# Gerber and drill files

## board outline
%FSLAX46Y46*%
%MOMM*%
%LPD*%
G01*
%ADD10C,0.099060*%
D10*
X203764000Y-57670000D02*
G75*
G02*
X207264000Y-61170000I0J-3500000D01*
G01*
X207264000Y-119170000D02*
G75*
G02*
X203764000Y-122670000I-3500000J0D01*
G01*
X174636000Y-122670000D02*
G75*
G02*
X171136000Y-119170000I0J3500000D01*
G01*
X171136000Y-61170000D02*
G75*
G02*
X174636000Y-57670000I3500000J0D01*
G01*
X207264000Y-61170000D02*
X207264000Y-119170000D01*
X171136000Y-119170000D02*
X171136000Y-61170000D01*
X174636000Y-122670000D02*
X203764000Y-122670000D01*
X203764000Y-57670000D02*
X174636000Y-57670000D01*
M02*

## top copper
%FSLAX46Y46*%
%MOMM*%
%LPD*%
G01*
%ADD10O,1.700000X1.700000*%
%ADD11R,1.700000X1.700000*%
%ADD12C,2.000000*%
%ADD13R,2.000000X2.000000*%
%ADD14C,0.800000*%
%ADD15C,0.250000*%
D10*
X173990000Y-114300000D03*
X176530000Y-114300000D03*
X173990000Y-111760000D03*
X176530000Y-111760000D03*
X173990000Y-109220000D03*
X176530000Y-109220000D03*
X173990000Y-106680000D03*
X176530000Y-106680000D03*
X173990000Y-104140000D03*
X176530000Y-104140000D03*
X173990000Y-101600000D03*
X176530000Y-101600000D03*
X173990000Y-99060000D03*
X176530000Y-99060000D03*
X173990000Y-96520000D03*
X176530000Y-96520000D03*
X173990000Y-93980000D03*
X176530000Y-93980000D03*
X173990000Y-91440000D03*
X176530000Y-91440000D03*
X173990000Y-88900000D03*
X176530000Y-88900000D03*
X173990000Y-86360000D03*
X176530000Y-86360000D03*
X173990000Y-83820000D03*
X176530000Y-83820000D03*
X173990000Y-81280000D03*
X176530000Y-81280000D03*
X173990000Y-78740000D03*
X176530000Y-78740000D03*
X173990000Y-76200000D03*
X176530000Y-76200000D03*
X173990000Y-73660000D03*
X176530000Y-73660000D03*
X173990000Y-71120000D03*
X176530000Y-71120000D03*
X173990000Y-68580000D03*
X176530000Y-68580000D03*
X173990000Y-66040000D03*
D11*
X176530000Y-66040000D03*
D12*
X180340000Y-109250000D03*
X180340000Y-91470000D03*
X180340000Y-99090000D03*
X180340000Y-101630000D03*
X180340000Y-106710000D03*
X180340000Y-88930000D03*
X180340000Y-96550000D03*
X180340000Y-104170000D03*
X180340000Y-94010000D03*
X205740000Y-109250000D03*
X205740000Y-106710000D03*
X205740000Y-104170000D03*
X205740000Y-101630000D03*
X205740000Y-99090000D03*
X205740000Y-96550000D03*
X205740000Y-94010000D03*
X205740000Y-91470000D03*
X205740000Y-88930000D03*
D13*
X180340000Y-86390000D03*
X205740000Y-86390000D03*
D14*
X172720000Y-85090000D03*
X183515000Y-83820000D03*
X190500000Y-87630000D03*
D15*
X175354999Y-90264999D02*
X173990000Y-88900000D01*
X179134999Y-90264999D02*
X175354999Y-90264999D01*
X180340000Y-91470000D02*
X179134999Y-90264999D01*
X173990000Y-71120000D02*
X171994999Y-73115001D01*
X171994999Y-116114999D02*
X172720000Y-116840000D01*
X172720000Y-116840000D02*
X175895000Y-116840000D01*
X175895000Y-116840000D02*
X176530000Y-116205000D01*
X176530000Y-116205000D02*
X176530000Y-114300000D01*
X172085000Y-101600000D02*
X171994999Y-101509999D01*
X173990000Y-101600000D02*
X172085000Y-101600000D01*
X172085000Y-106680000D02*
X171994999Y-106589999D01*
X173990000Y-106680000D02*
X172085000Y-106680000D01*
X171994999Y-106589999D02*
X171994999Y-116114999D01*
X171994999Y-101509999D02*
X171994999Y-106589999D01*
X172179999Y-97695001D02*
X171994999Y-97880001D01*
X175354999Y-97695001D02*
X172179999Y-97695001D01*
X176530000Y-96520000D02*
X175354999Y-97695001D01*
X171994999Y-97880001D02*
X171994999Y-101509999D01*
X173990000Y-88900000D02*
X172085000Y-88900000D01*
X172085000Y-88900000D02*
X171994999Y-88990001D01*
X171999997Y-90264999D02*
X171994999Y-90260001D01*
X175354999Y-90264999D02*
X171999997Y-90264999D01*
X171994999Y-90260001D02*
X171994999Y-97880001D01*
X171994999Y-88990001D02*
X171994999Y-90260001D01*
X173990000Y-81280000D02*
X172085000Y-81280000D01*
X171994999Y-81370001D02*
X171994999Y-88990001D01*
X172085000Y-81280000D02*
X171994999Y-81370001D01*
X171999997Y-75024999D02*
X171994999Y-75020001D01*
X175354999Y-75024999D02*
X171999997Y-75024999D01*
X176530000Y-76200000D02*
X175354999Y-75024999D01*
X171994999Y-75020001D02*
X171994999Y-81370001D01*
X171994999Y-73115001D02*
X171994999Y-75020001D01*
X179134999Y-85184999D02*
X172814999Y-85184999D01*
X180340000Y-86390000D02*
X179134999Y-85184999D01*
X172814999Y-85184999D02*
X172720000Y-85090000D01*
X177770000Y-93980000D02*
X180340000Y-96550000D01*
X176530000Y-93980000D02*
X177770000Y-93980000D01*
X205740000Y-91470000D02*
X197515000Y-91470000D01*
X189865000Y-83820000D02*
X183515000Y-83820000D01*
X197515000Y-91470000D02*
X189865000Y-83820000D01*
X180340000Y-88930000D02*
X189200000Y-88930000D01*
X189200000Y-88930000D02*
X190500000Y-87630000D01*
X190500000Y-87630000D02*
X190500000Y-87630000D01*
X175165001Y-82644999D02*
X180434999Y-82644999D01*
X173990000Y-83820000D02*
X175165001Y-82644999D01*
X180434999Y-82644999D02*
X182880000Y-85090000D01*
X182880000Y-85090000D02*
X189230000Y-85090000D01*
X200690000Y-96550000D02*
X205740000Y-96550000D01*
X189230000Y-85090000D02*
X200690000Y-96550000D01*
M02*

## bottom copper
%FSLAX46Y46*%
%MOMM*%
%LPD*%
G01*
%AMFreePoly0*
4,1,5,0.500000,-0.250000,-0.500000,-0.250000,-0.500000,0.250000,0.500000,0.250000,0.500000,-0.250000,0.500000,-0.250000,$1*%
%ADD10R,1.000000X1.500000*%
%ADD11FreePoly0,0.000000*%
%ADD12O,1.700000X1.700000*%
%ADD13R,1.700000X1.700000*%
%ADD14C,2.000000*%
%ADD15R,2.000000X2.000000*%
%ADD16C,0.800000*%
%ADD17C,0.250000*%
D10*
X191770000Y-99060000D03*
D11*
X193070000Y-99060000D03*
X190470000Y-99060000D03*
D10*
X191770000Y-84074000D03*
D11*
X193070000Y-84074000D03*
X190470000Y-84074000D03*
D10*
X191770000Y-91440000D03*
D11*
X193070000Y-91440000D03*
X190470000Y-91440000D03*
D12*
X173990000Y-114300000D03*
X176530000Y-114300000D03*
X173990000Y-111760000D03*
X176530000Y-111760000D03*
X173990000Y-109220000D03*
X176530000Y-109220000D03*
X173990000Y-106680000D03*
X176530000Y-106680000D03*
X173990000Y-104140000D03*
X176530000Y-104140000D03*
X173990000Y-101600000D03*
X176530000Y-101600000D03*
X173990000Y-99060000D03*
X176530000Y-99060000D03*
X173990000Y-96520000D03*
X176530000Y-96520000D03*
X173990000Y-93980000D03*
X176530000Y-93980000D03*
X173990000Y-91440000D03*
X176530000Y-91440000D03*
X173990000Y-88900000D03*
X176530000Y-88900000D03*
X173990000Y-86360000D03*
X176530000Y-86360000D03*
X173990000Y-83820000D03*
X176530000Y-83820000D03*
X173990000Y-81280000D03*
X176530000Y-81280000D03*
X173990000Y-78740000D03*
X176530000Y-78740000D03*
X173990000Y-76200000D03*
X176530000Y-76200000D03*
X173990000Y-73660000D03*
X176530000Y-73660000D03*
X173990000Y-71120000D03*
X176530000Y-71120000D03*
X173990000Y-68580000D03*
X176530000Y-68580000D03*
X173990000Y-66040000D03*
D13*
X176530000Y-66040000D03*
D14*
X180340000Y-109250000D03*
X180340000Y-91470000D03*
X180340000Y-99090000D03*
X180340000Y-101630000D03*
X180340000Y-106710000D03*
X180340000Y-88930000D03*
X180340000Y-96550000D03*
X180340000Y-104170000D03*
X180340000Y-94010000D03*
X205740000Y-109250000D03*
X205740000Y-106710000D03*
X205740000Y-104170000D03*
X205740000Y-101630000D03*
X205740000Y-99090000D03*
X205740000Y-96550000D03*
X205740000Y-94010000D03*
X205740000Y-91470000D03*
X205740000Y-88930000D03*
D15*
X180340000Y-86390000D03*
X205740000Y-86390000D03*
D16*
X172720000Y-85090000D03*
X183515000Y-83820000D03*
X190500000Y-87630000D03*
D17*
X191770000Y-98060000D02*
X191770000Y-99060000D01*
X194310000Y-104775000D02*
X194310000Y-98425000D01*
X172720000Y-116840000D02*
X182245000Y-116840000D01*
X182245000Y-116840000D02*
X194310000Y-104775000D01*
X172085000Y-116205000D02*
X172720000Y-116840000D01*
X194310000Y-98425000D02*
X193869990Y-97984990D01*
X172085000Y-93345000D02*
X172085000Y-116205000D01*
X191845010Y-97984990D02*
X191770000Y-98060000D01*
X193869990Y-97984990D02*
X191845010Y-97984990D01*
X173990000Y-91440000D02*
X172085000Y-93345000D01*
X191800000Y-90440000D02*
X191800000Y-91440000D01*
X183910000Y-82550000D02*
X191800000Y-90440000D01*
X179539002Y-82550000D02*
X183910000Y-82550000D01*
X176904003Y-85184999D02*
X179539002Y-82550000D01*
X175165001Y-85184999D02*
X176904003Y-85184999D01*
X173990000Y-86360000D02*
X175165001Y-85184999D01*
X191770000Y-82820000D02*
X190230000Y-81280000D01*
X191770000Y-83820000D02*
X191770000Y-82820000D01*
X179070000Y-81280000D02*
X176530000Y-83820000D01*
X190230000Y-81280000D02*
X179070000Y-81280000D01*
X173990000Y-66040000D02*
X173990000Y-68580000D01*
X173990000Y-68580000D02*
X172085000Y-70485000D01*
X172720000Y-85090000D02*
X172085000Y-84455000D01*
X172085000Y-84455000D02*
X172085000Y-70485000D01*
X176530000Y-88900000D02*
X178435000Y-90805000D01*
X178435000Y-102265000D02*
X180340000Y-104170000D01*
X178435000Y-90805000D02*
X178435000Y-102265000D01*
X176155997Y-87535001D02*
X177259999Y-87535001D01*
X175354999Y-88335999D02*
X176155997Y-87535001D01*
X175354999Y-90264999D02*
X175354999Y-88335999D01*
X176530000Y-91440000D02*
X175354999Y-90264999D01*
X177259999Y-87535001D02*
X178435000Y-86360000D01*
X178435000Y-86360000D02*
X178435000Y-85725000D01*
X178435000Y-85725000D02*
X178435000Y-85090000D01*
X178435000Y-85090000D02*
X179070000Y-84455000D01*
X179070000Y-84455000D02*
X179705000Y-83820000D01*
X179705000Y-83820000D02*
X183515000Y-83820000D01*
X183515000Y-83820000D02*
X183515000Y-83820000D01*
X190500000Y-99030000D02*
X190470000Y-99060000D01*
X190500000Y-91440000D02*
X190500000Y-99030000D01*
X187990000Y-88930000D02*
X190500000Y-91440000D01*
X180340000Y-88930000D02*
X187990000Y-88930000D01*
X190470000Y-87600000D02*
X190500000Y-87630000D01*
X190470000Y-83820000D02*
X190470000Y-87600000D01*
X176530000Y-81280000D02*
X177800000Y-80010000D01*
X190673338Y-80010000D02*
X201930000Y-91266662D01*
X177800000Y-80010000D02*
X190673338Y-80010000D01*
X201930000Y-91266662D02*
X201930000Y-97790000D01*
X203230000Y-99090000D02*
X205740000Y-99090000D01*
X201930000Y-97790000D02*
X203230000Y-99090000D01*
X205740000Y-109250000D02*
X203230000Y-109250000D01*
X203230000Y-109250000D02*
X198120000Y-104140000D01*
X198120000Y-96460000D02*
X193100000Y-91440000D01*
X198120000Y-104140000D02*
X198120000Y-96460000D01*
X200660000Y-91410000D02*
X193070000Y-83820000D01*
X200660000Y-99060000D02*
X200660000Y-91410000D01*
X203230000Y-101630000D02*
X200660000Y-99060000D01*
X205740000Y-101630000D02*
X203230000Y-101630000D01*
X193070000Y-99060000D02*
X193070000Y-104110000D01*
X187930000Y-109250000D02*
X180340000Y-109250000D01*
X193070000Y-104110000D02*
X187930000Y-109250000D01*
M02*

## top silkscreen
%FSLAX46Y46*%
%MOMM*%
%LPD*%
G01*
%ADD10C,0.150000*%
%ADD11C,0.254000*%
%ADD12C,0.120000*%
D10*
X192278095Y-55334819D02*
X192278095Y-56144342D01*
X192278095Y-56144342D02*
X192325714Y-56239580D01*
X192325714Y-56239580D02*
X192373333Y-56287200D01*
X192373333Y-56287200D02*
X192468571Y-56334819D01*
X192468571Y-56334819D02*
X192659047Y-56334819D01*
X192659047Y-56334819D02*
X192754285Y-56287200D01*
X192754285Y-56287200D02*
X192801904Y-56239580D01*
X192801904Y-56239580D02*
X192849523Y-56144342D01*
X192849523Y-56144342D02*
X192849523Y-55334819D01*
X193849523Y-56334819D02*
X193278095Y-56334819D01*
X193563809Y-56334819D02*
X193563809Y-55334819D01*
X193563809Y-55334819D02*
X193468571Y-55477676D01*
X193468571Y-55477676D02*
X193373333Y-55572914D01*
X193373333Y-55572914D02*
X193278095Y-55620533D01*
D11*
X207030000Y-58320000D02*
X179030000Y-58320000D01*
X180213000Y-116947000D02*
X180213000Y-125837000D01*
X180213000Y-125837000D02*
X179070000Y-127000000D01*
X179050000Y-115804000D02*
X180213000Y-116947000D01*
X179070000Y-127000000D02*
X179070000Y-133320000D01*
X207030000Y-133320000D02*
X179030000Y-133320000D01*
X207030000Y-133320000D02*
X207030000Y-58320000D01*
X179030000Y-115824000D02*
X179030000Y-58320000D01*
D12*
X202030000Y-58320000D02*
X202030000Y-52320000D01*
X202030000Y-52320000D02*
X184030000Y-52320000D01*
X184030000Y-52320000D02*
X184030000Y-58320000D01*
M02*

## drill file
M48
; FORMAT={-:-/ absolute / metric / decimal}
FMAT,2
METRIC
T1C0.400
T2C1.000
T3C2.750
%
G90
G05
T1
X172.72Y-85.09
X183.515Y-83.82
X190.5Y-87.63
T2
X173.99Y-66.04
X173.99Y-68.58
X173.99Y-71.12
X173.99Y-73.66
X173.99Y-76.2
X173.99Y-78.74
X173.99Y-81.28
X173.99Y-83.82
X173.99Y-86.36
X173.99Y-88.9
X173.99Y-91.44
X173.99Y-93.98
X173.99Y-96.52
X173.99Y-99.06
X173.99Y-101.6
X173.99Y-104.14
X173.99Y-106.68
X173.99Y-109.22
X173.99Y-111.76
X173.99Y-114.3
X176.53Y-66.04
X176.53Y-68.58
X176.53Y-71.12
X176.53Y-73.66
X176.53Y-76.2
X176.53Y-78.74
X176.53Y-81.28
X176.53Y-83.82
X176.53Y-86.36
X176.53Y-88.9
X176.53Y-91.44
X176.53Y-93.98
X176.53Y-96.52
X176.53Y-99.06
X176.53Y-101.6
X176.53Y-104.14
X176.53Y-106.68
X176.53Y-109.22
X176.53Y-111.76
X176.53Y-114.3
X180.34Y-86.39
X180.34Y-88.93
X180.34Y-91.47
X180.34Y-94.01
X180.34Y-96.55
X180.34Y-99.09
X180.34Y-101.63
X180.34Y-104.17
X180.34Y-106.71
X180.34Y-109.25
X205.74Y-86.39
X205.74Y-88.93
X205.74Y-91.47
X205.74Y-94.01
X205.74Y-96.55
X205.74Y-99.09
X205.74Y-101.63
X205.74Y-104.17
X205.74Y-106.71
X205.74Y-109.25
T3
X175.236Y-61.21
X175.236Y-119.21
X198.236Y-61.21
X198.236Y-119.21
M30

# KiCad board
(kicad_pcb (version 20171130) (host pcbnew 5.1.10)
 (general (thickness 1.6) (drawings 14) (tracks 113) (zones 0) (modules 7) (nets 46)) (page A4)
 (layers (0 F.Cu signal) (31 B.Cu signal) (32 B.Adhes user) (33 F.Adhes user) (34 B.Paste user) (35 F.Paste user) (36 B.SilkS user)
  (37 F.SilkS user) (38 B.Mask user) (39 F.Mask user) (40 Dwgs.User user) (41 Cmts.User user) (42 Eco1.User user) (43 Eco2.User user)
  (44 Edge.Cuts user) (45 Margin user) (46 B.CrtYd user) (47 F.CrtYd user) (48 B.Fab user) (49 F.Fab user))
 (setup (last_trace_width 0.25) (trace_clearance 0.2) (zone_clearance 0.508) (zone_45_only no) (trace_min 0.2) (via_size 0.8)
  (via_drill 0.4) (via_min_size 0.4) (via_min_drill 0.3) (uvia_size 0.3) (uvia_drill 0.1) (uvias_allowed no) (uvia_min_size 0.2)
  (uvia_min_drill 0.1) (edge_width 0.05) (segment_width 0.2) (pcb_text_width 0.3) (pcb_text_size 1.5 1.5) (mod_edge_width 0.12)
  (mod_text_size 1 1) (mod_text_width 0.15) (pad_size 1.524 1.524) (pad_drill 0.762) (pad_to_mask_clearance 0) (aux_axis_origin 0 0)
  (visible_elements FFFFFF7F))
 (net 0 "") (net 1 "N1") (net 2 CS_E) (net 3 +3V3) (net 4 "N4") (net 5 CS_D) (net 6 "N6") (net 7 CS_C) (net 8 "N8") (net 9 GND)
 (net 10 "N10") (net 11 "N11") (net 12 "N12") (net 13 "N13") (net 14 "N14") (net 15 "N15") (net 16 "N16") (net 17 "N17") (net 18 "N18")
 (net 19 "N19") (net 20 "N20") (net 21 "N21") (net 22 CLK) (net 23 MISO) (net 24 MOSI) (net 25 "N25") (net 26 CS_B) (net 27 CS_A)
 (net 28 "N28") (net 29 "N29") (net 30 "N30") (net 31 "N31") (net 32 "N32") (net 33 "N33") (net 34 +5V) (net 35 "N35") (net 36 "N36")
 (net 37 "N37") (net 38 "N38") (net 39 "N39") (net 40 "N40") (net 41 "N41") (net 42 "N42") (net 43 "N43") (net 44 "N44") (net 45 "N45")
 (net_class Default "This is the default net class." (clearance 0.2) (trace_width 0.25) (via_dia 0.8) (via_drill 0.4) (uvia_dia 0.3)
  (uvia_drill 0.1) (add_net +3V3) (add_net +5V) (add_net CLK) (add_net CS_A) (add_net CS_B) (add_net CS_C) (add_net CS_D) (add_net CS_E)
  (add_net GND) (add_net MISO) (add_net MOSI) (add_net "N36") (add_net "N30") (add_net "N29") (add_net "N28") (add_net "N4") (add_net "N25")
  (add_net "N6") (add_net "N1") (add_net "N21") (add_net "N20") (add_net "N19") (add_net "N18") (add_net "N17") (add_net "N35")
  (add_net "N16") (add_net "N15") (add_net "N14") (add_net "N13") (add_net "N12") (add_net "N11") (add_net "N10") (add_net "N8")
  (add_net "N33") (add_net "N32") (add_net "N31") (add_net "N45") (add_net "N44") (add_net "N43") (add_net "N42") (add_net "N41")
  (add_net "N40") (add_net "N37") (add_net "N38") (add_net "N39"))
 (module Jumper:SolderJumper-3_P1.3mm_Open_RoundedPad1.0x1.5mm (layer B.Cu) (at 191.77 99.06)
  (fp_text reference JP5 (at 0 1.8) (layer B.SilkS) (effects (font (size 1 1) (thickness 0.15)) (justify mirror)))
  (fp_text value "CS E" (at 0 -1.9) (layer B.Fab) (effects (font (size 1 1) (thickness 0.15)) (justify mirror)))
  (pad 2 smd rect (at 0 0) (size 1 1.5) (layers B.Cu B.Mask) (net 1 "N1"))
  (pad 3 smd custom (at 1.3 0) (size 1 0.5) (layers B.Cu B.Mask) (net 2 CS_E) (zone_connect 2) (options (clearance outline) (anchor rect))
   (primitives))
  (pad 1 smd custom (at -1.3 0) (size 1 0.5) (layers B.Cu B.Mask) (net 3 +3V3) (zone_connect 2) (options (clearance outline) (anchor rect))
   (primitives)))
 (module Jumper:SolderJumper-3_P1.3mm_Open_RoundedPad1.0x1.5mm (layer B.Cu) (at 191.77 84.074)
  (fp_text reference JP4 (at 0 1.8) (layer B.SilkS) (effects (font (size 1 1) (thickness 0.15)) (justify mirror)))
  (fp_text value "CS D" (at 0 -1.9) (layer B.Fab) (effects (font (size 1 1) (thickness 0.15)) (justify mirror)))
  (pad 2 smd rect (at 0 0) (size 1 1.5) (layers B.Cu B.Mask) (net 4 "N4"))
  (pad 3 smd custom (at 1.3 0) (size 1 0.5) (layers B.Cu B.Mask) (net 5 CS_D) (zone_connect 2) (options (clearance outline) (anchor rect))
   (primitives))
  (pad 1 smd custom (at -1.3 0) (size 1 0.5) (layers B.Cu B.Mask) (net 3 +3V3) (zone_connect 2) (options (clearance outline) (anchor rect))
   (primitives)))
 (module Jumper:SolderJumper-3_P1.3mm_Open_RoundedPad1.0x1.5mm (layer B.Cu) (at 191.77 91.44)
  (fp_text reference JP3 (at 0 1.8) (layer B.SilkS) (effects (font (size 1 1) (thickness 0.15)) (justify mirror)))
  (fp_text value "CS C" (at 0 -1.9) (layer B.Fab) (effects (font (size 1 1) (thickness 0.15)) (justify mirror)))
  (pad 2 smd rect (at 0 0) (size 1 1.5) (layers B.Cu B.Mask) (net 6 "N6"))
  (pad 3 smd custom (at 1.3 0) (size 1 0.5) (layers B.Cu B.Mask) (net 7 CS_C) (zone_connect 2) (options (clearance outline) (anchor rect))
   (primitives))
  (pad 1 smd custom (at -1.3 0) (size 1 0.5) (layers B.Cu B.Mask) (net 3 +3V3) (zone_connect 2) (options (clearance outline) (anchor rect))
   (primitives)))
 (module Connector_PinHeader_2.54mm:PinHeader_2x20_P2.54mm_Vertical (layer B.Cu) (at 176.53 66.04 180)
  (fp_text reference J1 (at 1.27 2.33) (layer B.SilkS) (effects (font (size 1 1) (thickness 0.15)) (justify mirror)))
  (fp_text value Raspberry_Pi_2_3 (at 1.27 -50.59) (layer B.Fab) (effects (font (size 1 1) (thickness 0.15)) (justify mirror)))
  (pad 40 thru_hole oval (at 2.54 -48.26 180) (size 1.7 1.7) (drill 1) (layers *.Cu *.Mask) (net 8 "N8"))
  (pad 39 thru_hole oval (at 0 -48.26 180) (size 1.7 1.7) (drill 1) (layers *.Cu *.Mask) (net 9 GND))
  (pad 38 thru_hole oval (at 2.54 -45.72 180) (size 1.7 1.7) (drill 1) (layers *.Cu *.Mask) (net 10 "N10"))
  (pad 37 thru_hole oval (at 0 -45.72 180) (size 1.7 1.7) (drill 1) (layers *.Cu *.Mask) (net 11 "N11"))
  (pad 36 thru_hole oval (at 2.54 -43.18 180) (size 1.7 1.7) (drill 1) (layers *.Cu *.Mask) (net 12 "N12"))
  (pad 35 thru_hole oval (at 0 -43.18 180) (size 1.7 1.7) (drill 1) (layers *.Cu *.Mask) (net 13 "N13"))
  (pad 34 thru_hole oval (at 2.54 -40.64 180) (size 1.7 1.7) (drill 1) (layers *.Cu *.Mask) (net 9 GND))
  (pad 33 thru_hole oval (at 0 -40.64 180) (size 1.7 1.7) (drill 1) (layers *.Cu *.Mask) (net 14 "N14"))
  (pad 32 thru_hole oval (at 2.54 -38.1 180) (size 1.7 1.7) (drill 1) (layers *.Cu *.Mask) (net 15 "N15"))
  (pad 31 thru_hole oval (at 0 -38.1 180) (size 1.7 1.7) (drill 1) (layers *.Cu *.Mask) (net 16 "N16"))
  (pad 30 thru_hole oval (at 2.54 -35.56 180) (size 1.7 1.7) (drill 1) (layers *.Cu *.Mask) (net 9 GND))
  (pad 29 thru_hole oval (at 0 -35.56 180) (size 1.7 1.7) (drill 1) (layers *.Cu *.Mask) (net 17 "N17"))
  (pad 28 thru_hole oval (at 2.54 -33.02 180) (size 1.7 1.7) (drill 1) (layers *.Cu *.Mask) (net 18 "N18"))
  (pad 27 thru_hole oval (at 0 -33.02 180) (size 1.7 1.7) (drill 1) (layers *.Cu *.Mask) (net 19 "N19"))
  (pad 26 thru_hole oval (at 2.54 -30.48 180) (size 1.7 1.7) (drill 1) (layers *.Cu *.Mask) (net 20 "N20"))
  (pad 25 thru_hole oval (at 0 -30.48 180) (size 1.7 1.7) (drill 1) (layers *.Cu *.Mask) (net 9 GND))
  (pad 24 thru_hole oval (at 2.54 -27.94 180) (size 1.7 1.7) (drill 1) (layers *.Cu *.Mask) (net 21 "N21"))
  (pad 23 thru_hole oval (at 0 -27.94 180) (size 1.7 1.7) (drill 1) (layers *.Cu *.Mask) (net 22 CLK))
  (pad 22 thru_hole oval (at 2.54 -25.4 180) (size 1.7 1.7) (drill 1) (layers *.Cu *.Mask) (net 1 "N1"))
  (pad 21 thru_hole oval (at 0 -25.4 180) (size 1.7 1.7) (drill 1) (layers *.Cu *.Mask) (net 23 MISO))
  (pad 20 thru_hole oval (at 2.54 -22.86 180) (size 1.7 1.7) (drill 1) (layers *.Cu *.Mask) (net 9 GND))
  (pad 19 thru_hole oval (at 0 -22.86 180) (size 1.7 1.7) (drill 1) (layers *.Cu *.Mask) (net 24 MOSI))
  (pad 18 thru_hole oval (at 2.54 -20.32 180) (size 1.7 1.7) (drill 1) (layers *.Cu *.Mask) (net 6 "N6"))
  (pad 17 thru_hole oval (at 0 -20.32 180) (size 1.7 1.7) (drill 1) (layers *.Cu *.Mask) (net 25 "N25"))
  (pad 16 thru_hole oval (at 2.54 -17.78 180) (size 1.7 1.7) (drill 1) (layers *.Cu *.Mask) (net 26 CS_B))
  (pad 15 thru_hole oval (at 0 -17.78 180) (size 1.7 1.7) (drill 1) (layers *.Cu *.Mask) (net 4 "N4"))
  (pad 14 thru_hole oval (at 2.54 -15.24 180) (size 1.7 1.7) (drill 1) (layers *.Cu *.Mask) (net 9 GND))
  (pad 13 thru_hole oval (at 0 -15.24 180) (size 1.7 1.7) (drill 1) (layers *.Cu *.Mask) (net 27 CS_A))
  (pad 12 thru_hole oval (at 2.54 -12.7 180) (size 1.7 1.7) (drill 1) (layers *.Cu *.Mask) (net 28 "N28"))
  (pad 11 thru_hole oval (at 0 -12.7 180) (size 1.7 1.7) (drill 1) (layers *.Cu *.Mask) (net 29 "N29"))
  (pad 10 thru_hole oval (at 2.54 -10.16 180) (size 1.7 1.7) (drill 1) (layers *.Cu *.Mask) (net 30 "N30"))
  (pad 9 thru_hole oval (at 0 -10.16 180) (size 1.7 1.7) (drill 1) (layers *.Cu *.Mask) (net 9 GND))
  (pad 8 thru_hole oval (at 2.54 -7.62 180) (size 1.7 1.7) (drill 1) (layers *.Cu *.Mask) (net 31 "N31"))
  (pad 7 thru_hole oval (at 0 -7.62 180) (size 1.7 1.7) (drill 1) (layers *.Cu *.Mask) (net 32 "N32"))
  (pad 6 thru_hole oval (at 2.54 -5.08 180) (size 1.7 1.7) (drill 1) (layers *.Cu *.Mask) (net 9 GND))
  (pad 5 thru_hole oval (at 0 -5.08 180) (size 1.7 1.7) (drill 1) (layers *.Cu *.Mask) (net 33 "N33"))
  (pad 4 thru_hole oval (at 2.54 -2.54 180) (size 1.7 1.7) (drill 1) (layers *.Cu *.Mask) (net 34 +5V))
  (pad 3 thru_hole oval (at 0 -2.54 180) (size 1.7 1.7) (drill 1) (layers *.Cu *.Mask) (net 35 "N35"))
  (pad 2 thru_hole oval (at 2.54 0 180) (size 1.7 1.7) (drill 1) (layers *.Cu *.Mask) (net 34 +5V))
  (pad 1 thru_hole rect (at 0 0 180) (size 1.7 1.7) (drill 1) (layers *.Cu *.Mask) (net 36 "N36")))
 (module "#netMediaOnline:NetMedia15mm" (layer B.Cu) (at 192.405 71.755 180)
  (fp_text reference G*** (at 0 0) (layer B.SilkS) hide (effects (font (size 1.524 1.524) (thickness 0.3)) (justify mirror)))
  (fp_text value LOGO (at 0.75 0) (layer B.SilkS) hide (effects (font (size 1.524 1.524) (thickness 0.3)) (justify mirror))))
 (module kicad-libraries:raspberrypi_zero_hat (layer B.Cu) (at 175.236 90.21 270)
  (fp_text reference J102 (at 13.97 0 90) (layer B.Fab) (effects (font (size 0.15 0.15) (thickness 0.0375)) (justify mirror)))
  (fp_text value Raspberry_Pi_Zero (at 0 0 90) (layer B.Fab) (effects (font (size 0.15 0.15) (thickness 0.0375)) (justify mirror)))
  (pad "" np_thru_hole circle (at -29 -23 270) (size 2.75 2.75) (drill 2.75) (layers *.Cu *.Mask B.SilkS))
  (pad "" np_thru_hole circle (at 29 -23 270) (size 2.75 2.75) (drill 2.75) (layers *.Cu *.Mask B.SilkS))
  (pad "" np_thru_hole circle (at -29 0 270) (size 2.75 2.75) (drill 2.75) (layers *.Cu *.Mask B.SilkS))
  (pad "" np_thru_hole circle (at 29 0 270) (size 2.75 2.75) (drill 2.75) (layers *.Cu *.Mask B.SilkS)))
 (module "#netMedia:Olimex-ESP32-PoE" (layer F.Cu) (at 180.34 86.36)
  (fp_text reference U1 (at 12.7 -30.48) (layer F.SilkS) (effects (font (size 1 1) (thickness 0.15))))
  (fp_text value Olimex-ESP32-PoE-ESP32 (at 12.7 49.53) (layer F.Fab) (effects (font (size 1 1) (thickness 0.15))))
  (fp_line (start 26.69 -28.04) (end -1.31 -28.04) (layer F.SilkS) (width 0.254))
  (fp_line (start -0.127 30.587) (end -0.127 39.477) (layer F.SilkS) (width 0.254))
  (fp_line (start -0.127 39.477) (end -1.27 40.64) (layer F.SilkS) (width 0.254))
  (fp_line (start -1.29 29.444) (end -0.127 30.587) (layer F.SilkS) (width 0.254))
  (fp_line (start -1.27 40.64) (end -1.27 46.96) (layer F.SilkS) (width 0.254))
  (fp_line (start 26.69 46.96) (end -1.31 46.96) (layer F.SilkS) (width 0.254))
  (fp_line (start 26.69 46.96) (end 26.69 -28.04) (layer F.SilkS) (width 0.254))
  (fp_line (start -1.31 29.464) (end -1.31 -28.04) (layer F.SilkS) (width 0.254))
  (fp_line (start 21.69 -28.04) (end 21.69 -34.04) (layer F.SilkS) (width 0.12))
  (fp_line (start 21.69 -34.04) (end 3.69 -34.04) (layer F.SilkS) (width 0.12))
  (fp_line (start 3.69 -34.04) (end 3.69 -28.04) (layer F.SilkS) (width 0.12))
  (pad 10 thru_hole circle (at 0 22.89) (size 2 2) (drill 1) (layers *.Cu *.Mask) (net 2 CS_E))
  (pad 3 thru_hole circle (at 0 5.11) (size 2 2) (drill 1) (layers *.Cu *.Mask) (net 9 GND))
  (pad 6 thru_hole circle (at 0 12.73) (size 2 2) (drill 1) (layers *.Cu *.Mask) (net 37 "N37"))
  (pad 7 thru_hole circle (at 0 15.27) (size 2 2) (drill 1) (layers *.Cu *.Mask) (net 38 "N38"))
  (pad 9 thru_hole circle (at 0 20.35) (size 2 2) (drill 1) (layers *.Cu *.Mask) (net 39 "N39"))
  (pad 2 thru_hole circle (at 0 2.57) (size 2 2) (drill 1) (layers *.Cu *.Mask) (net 3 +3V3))
  (pad 5 thru_hole circle (at 0 10.19) (size 2 2) (drill 1) (layers *.Cu *.Mask) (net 22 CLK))
  (pad 8 thru_hole circle (at 0 17.81) (size 2 2) (drill 1) (layers *.Cu *.Mask) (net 24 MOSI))
  (pad 4 thru_hole circle (at 0 7.65) (size 2 2) (drill 1) (layers *.Cu *.Mask) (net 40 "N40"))
  (pad 20 thru_hole circle (at 25.4 22.89) (size 2 2) (drill 1) (layers *.Cu *.Mask) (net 7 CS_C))
  (pad 19 thru_hole circle (at 25.4 20.35) (size 2 2) (drill 1) (layers *.Cu *.Mask) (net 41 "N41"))
  (pad 18 thru_hole circle (at 25.4 17.81) (size 2 2) (drill 1) (layers *.Cu *.Mask) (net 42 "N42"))
  (pad 17 thru_hole circle (at 25.4 15.27) (size 2 2) (drill 1) (layers *.Cu *.Mask) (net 5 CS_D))
  (pad 16 thru_hole circle (at 25.4 12.73) (size 2 2) (drill 1) (layers *.Cu *.Mask) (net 27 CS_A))
  (pad 15 thru_hole circle (at 25.4 10.19) (size 2 2) (drill 1) (layers *.Cu *.Mask) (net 26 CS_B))
  (pad 14 thru_hole circle (at 25.4 7.65) (size 2 2) (drill 1) (layers *.Cu *.Mask) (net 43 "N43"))
  (pad 13 thru_hole circle (at 25.4 5.11) (size 2 2) (drill 1) (layers *.Cu *.Mask) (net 23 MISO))
  (pad 12 thru_hole circle (at 25.4 2.57) (size 2 2) (drill 1) (layers *.Cu *.Mask) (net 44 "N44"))
  (pad 1 thru_hole rect (at 0 0.03) (size 2 2) (drill 1) (layers *.Cu *.Mask) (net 34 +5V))
  (pad 11 thru_hole rect (at 25.4 0.03 90) (size 2 2) (drill 1) (layers *.Cu *.Mask) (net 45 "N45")))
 (gr_arc (start 203.764 61.17) (end 203.764 57.67) (angle 90) (layer Edge.Cuts) (width 0.09906))
 (gr_arc (start 203.764 119.17) (end 207.264 119.17) (angle 90) (layer Edge.Cuts) (width 0.09906))
 (gr_arc (start 174.636 119.17) (end 174.636 122.67) (angle 90) (layer Edge.Cuts) (width 0.09906))
 (gr_arc (start 174.636 61.17) (end 171.136 61.17) (angle 90) (layer Edge.Cuts) (width 0.09906))
 (gr_line (start 207.264 61.17) (end 207.264 119.17) (angle 90) (layer Edge.Cuts) (width 0.09906))
 (gr_line (start 171.136 119.17) (end 171.136 61.17) (angle 90) (layer Edge.Cuts) (width 0.09906))
 (gr_line (start 174.636 122.67) (end 203.764 122.67) (angle 90) (layer Edge.Cuts) (width 0.09906))
 (gr_line (start 203.764 57.67) (end 174.636 57.67) (angle 90) (layer Edge.Cuts) (width 0.09906))
 (segment (start 175.354999 90.264999) (end 173.99 88.9) (width 0.25) (layer F.Cu) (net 9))
 (segment (start 179.134999 90.264999) (end 175.354999 90.264999) (width 0.25) (layer F.Cu) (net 9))
 (segment (start 180.34 91.47) (end 179.134999 90.264999) (width 0.25) (layer F.Cu) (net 9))
 (segment (start 173.99 71.12) (end 171.994999 73.115001) (width 0.25) (layer F.Cu) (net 9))
 (segment (start 171.994999 116.114999) (end 172.72 116.84) (width 0.25) (layer F.Cu) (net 9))
 (segment (start 172.72 116.84) (end 175.895 116.84) (width 0.25) (layer F.Cu) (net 9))
 (segment (start 175.895 116.84) (end 176.53 116.205) (width 0.25) (layer F.Cu) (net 9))
 (segment (start 176.53 116.205) (end 176.53 114.3) (width 0.25) (layer F.Cu) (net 9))
 (segment (start 172.085 101.6) (end 171.994999 101.509999) (width 0.25) (layer F.Cu) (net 9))
 (segment (start 173.99 101.6) (end 172.085 101.6) (width 0.25) (layer F.Cu) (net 9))
 (segment (start 172.085 106.68) (end 171.994999 106.589999) (width 0.25) (layer F.Cu) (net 9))
 (segment (start 173.99 106.68) (end 172.085 106.68) (width 0.25) (layer F.Cu) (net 9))
 (segment (start 171.994999 106.589999) (end 171.994999 116.114999) (width 0.25) (layer F.Cu) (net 9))
 (segment (start 171.994999 101.509999) (end 171.994999 106.589999) (width 0.25) (layer F.Cu) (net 9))
 (segment (start 172.179999 97.695001) (end 171.994999 97.880001) (width 0.25) (layer F.Cu) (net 9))
 (segment (start 175.354999 97.695001) (end 172.179999 97.695001) (width 0.25) (layer F.Cu) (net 9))
 (segment (start 176.53 96.52) (end 175.354999 97.695001) (width 0.25) (layer F.Cu) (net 9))
 (segment (start 171.994999 97.880001) (end 171.994999 101.509999) (width 0.25) (layer F.Cu) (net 9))
 (segment (start 173.99 88.9) (end 172.085 88.9) (width 0.25) (layer F.Cu) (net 9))
 (segment (start 172.085 88.9) (end 171.994999 88.990001) (width 0.25) (layer F.Cu) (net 9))
 (segment (start 171.999997 90.264999) (end 171.994999 90.260001) (width 0.25) (layer F.Cu) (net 9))
 (segment (start 175.354999 90.264999) (end 171.999997 90.264999) (width 0.25) (layer F.Cu) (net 9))
 (segment (start 171.994999 90.260001) (end 171.994999 97.880001) (width 0.25) (layer F.Cu) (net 9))
 (segment (start 171.994999 88.990001) (end 171.994999 90.260001) (width 0.25) (layer F.Cu) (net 9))
 (segment (start 173.99 81.28) (end 172.085 81.28) (width 0.25) (layer F.Cu) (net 9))
 (segment (start 171.994999 81.370001) (end 171.994999 88.990001) (width 0.25) (layer F.Cu) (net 9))
 (segment (start 172.085 81.28) (end 171.994999 81.370001) (width 0.25) (layer F.Cu) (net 9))
 (segment (start 171.999997 75.024999) (end 171.994999 75.020001) (width 0.25) (layer F.Cu) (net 9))
 (segment (start 175.354999 75.024999) (end 171.999997 75.024999) (width 0.25) (layer F.Cu) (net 9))
 (segment (start 176.53 76.2) (end 175.354999 75.024999) (width 0.25) (layer F.Cu) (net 9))
 (segment (start 171.994999 75.020001) (end 171.994999 81.370001) (width 0.25) (layer F.Cu) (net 9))
 (segment (start 171.994999 73.115001) (end 171.994999 75.020001) (width 0.25) (layer F.Cu) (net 9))
 (segment (start 191.77 98.06) (end 191.77 99.06) (width 0.25) (layer B.Cu) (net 1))
 (segment (start 194.31 104.775) (end 194.31 98.425) (width 0.25) (layer B.Cu) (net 1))
 (segment (start 172.72 116.84) (end 182.245 116.84) (width 0.25) (layer B.Cu) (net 1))
 (segment (start 182.245 116.84) (end 194.31 104.775) (width 0.25) (layer B.Cu) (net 1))
 (segment (start 172.085 116.205) (end 172.72 116.84) (width 0.25) (layer B.Cu) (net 1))
 (segment (start 194.31 98.425) (end 193.86999 97.98499) (width 0.25) (layer B.Cu) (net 1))
 (segment (start 172.085 93.345) (end 172.085 116.205) (width 0.25) (layer B.Cu) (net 1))
 (segment (start 191.84501 97.98499) (end 191.77 98.06) (width 0.25) (layer B.Cu) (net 1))
 (segment (start 193.86999 97.98499) (end 191.84501 97.98499) (width 0.25) (layer B.Cu) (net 1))
 (segment (start 173.99 91.44) (end 172.085 93.345) (width 0.25) (layer B.Cu) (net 1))
 (segment (start 191.8 90.44) (end 191.8 91.44) (width 0.25) (layer B.Cu) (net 6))
 (segment (start 183.91 82.55) (end 191.8 90.44) (width 0.25) (layer B.Cu) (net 6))
 (segment (start 179.539002 82.55) (end 183.91 82.55) (width 0.25) (layer B.Cu) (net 6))
 (segment (start 176.904003 85.184999) (end 179.539002 82.55) (width 0.25) (layer B.Cu) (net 6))
 (segment (start 175.165001 85.184999) (end 176.904003 85.184999) (width 0.25) (layer B.Cu) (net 6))
 (segment (start 173.99 86.36) (end 175.165001 85.184999) (width 0.25) (layer B.Cu) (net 6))
 (segment (start 191.77 82.82) (end 190.23 81.28) (width 0.25) (layer B.Cu) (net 4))
 (segment (start 191.77 83.82) (end 191.77 82.82) (width 0.25) (layer B.Cu) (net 4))
 (segment (start 179.07 81.28) (end 176.53 83.82) (width 0.25) (layer B.Cu) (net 4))
 (segment (start 190.23 81.28) (end 179.07 81.28) (width 0.25) (layer B.Cu) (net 4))
 (segment (start 179.134999 85.184999) (end 172.814999 85.184999) (width 0.25) (layer F.Cu) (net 34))
 (segment (start 180.34 86.39) (end 179.134999 85.184999) (width 0.25) (layer F.Cu) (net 34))
 (segment (start 172.814999 85.184999) (end 172.72 85.09) (width 0.25) (layer F.Cu) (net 34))
 (segment (start 173.99 66.04) (end 173.99 68.58) (width 0.25) (layer B.Cu) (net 34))
 (segment (start 173.99 68.58) (end 172.085 70.485) (width 0.25) (layer B.Cu) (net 34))
 (via (at 172.72 85.09) (size 0.8) (drill 0.4) (layers F.Cu B.Cu) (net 34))
 (segment (start 172.72 85.09) (end 172.085 84.455) (width 0.25) (layer B.Cu) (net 34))
 (segment (start 172.085 84.455) (end 172.085 70.485) (width 0.25) (layer B.Cu) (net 34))
 (segment (start 177.77 93.98) (end 180.34 96.55) (width 0.25) (layer F.Cu) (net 22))
 (segment (start 176.53 93.98) (end 177.77 93.98) (width 0.25) (layer F.Cu) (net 22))
 (segment (start 176.53 88.9) (end 178.435 90.805) (width 0.25) (layer B.Cu) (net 24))
 (segment (start 178.435 102.265) (end 180.34 104.17) (width 0.25) (layer B.Cu) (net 24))
 (segment (start 178.435 90.805) (end 178.435 102.265) (width 0.25) (layer B.Cu) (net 24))
 (segment (start 176.155997 87.535001) (end 177.259999 87.535001) (width 0.25) (layer B.Cu) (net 23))
 (segment (start 175.354999 88.335999) (end 176.155997 87.535001) (width 0.25) (layer B.Cu) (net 23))
 (segment (start 175.354999 90.264999) (end 175.354999 88.335999) (width 0.25) (layer B.Cu) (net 23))
 (segment (start 176.53 91.44) (end 175.354999 90.264999) (width 0.25) (layer B.Cu) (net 23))
 (segment (start 177.259999 87.535001) (end 178.435 86.36) (width 0.25) (layer B.Cu) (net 23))
 (segment (start 178.435 86.36) (end 178.435 85.725) (width 0.25) (layer B.Cu) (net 23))
 (segment (start 178.435 85.725) (end 178.435 85.09) (width 0.25) (layer B.Cu) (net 23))
 (segment (start 178.435 85.09) (end 179.07 84.455) (width 0.25) (layer B.Cu) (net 23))
 (segment (start 179.07 84.455) (end 179.705 83.82) (width 0.25) (layer B.Cu) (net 23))
 (segment (start 179.705 83.82) (end 183.515 83.82) (width 0.25) (layer B.Cu) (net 23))
 (segment (start 183.515 83.82) (end 183.515 83.82) (width 0.25) (layer B.Cu) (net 23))
 (via (at 183.515 83.82) (size 0.8) (drill 0.4) (layers F.Cu B.Cu) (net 23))
 (segment (start 205.74 91.47) (end 197.515 91.47) (width 0.25) (layer F.Cu) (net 23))
 (segment (start 189.865 83.82) (end 183.515 83.82) (width 0.25) (layer F.Cu) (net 23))
 (segment (start 197.515 91.47) (end 189.865 83.82) (width 0.25) (layer F.Cu) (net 23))
 (segment (start 190.5 99.03) (end 190.47 99.06) (width 0.25) (layer B.Cu) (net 3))
 (segment (start 190.5 91.44) (end 190.5 99.03) (width 0.25) (layer B.Cu) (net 3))
 (segment (start 187.99 88.93) (end 190.5 91.44) (width 0.25) (layer B.Cu) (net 3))
 (segment (start 180.34 88.93) (end 187.99 88.93) (width 0.25) (layer B.Cu) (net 3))
 (segment (start 180.34 88.93) (end 189.2 88.93) (width 0.25) (layer F.Cu) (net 3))
 (segment (start 189.2 88.93) (end 190.5 87.63) (width 0.25) (layer F.Cu) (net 3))
 (segment (start 190.5 87.63) (end 190.5 87.63) (width 0.25) (layer F.Cu) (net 3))
 (via (at 190.5 87.63) (size 0.8) (drill 0.4) (layers F.Cu B.Cu) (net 3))
 (segment (start 190.47 87.6) (end 190.5 87.63) (width 0.25) (layer B.Cu) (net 3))
 (segment (start 190.47 83.82) (end 190.47 87.6) (width 0.25) (layer B.Cu) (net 3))
 (segment (start 176.53 81.28) (end 177.8 80.01) (width 0.25) (layer B.Cu) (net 27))
 (segment (start 190.673338 80.01) (end 201.93 91.266662) (width 0.25) (layer B.Cu) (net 27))
 (segment (start 177.8 80.01) (end 190.673338 80.01) (width 0.25) (layer B.Cu) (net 27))
 (segment (start 201.93 91.266662) (end 201.93 97.79) (width 0.25) (layer B.Cu) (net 27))
 (segment (start 203.23 99.09) (end 205.74 99.09) (width 0.25) (layer B.Cu) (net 27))
 (segment (start 201.93 97.79) (end 203.23 99.09) (width 0.25) (layer B.Cu) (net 27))
 (segment (start 175.165001 82.644999) (end 180.434999 82.644999) (width 0.25) (layer F.Cu) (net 26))
 (segment (start 173.99 83.82) (end 175.165001 82.644999) (width 0.25) (layer F.Cu) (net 26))
 (segment (start 180.434999 82.644999) (end 182.88 85.09) (width 0.25) (layer F.Cu) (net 26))
 (segment (start 182.88 85.09) (end 189.23 85.09) (width 0.25) (layer F.Cu) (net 26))
 (segment (start 200.69 96.55) (end 205.74 96.55) (width 0.25) (layer F.Cu) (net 26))
 (segment (start 189.23 85.09) (end 200.69 96.55) (width 0.25) (layer F.Cu) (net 26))
 (segment (start 205.74 109.25) (end 203.23 109.25) (width 0.25) (layer B.Cu) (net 7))
 (segment (start 203.23 109.25) (end 198.12 104.14) (width 0.25) (layer B.Cu) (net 7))
 (segment (start 198.12 96.46) (end 193.1 91.44) (width 0.25) (layer B.Cu) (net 7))
 (segment (start 198.12 104.14) (end 198.12 96.46) (width 0.25) (layer B.Cu) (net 7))
 (segment (start 200.66 91.41) (end 193.07 83.82) (width 0.25) (layer B.Cu) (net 5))
 (segment (start 200.66 99.06) (end 200.66 91.41) (width 0.25) (layer B.Cu) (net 5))
 (segment (start 203.23 101.63) (end 200.66 99.06) (width 0.25) (layer B.Cu) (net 5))
 (segment (start 205.74 101.63) (end 203.23 101.63) (width 0.25) (layer B.Cu) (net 5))
 (segment (start 193.07 99.06) (end 193.07 104.11) (width 0.25) (layer B.Cu) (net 2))
 (segment (start 187.93 109.25) (end 180.34 109.25) (width 0.25) (layer B.Cu) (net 2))
 (segment (start 193.07 104.11) (end 187.93 109.25) (width 0.25) (layer B.Cu) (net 2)))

